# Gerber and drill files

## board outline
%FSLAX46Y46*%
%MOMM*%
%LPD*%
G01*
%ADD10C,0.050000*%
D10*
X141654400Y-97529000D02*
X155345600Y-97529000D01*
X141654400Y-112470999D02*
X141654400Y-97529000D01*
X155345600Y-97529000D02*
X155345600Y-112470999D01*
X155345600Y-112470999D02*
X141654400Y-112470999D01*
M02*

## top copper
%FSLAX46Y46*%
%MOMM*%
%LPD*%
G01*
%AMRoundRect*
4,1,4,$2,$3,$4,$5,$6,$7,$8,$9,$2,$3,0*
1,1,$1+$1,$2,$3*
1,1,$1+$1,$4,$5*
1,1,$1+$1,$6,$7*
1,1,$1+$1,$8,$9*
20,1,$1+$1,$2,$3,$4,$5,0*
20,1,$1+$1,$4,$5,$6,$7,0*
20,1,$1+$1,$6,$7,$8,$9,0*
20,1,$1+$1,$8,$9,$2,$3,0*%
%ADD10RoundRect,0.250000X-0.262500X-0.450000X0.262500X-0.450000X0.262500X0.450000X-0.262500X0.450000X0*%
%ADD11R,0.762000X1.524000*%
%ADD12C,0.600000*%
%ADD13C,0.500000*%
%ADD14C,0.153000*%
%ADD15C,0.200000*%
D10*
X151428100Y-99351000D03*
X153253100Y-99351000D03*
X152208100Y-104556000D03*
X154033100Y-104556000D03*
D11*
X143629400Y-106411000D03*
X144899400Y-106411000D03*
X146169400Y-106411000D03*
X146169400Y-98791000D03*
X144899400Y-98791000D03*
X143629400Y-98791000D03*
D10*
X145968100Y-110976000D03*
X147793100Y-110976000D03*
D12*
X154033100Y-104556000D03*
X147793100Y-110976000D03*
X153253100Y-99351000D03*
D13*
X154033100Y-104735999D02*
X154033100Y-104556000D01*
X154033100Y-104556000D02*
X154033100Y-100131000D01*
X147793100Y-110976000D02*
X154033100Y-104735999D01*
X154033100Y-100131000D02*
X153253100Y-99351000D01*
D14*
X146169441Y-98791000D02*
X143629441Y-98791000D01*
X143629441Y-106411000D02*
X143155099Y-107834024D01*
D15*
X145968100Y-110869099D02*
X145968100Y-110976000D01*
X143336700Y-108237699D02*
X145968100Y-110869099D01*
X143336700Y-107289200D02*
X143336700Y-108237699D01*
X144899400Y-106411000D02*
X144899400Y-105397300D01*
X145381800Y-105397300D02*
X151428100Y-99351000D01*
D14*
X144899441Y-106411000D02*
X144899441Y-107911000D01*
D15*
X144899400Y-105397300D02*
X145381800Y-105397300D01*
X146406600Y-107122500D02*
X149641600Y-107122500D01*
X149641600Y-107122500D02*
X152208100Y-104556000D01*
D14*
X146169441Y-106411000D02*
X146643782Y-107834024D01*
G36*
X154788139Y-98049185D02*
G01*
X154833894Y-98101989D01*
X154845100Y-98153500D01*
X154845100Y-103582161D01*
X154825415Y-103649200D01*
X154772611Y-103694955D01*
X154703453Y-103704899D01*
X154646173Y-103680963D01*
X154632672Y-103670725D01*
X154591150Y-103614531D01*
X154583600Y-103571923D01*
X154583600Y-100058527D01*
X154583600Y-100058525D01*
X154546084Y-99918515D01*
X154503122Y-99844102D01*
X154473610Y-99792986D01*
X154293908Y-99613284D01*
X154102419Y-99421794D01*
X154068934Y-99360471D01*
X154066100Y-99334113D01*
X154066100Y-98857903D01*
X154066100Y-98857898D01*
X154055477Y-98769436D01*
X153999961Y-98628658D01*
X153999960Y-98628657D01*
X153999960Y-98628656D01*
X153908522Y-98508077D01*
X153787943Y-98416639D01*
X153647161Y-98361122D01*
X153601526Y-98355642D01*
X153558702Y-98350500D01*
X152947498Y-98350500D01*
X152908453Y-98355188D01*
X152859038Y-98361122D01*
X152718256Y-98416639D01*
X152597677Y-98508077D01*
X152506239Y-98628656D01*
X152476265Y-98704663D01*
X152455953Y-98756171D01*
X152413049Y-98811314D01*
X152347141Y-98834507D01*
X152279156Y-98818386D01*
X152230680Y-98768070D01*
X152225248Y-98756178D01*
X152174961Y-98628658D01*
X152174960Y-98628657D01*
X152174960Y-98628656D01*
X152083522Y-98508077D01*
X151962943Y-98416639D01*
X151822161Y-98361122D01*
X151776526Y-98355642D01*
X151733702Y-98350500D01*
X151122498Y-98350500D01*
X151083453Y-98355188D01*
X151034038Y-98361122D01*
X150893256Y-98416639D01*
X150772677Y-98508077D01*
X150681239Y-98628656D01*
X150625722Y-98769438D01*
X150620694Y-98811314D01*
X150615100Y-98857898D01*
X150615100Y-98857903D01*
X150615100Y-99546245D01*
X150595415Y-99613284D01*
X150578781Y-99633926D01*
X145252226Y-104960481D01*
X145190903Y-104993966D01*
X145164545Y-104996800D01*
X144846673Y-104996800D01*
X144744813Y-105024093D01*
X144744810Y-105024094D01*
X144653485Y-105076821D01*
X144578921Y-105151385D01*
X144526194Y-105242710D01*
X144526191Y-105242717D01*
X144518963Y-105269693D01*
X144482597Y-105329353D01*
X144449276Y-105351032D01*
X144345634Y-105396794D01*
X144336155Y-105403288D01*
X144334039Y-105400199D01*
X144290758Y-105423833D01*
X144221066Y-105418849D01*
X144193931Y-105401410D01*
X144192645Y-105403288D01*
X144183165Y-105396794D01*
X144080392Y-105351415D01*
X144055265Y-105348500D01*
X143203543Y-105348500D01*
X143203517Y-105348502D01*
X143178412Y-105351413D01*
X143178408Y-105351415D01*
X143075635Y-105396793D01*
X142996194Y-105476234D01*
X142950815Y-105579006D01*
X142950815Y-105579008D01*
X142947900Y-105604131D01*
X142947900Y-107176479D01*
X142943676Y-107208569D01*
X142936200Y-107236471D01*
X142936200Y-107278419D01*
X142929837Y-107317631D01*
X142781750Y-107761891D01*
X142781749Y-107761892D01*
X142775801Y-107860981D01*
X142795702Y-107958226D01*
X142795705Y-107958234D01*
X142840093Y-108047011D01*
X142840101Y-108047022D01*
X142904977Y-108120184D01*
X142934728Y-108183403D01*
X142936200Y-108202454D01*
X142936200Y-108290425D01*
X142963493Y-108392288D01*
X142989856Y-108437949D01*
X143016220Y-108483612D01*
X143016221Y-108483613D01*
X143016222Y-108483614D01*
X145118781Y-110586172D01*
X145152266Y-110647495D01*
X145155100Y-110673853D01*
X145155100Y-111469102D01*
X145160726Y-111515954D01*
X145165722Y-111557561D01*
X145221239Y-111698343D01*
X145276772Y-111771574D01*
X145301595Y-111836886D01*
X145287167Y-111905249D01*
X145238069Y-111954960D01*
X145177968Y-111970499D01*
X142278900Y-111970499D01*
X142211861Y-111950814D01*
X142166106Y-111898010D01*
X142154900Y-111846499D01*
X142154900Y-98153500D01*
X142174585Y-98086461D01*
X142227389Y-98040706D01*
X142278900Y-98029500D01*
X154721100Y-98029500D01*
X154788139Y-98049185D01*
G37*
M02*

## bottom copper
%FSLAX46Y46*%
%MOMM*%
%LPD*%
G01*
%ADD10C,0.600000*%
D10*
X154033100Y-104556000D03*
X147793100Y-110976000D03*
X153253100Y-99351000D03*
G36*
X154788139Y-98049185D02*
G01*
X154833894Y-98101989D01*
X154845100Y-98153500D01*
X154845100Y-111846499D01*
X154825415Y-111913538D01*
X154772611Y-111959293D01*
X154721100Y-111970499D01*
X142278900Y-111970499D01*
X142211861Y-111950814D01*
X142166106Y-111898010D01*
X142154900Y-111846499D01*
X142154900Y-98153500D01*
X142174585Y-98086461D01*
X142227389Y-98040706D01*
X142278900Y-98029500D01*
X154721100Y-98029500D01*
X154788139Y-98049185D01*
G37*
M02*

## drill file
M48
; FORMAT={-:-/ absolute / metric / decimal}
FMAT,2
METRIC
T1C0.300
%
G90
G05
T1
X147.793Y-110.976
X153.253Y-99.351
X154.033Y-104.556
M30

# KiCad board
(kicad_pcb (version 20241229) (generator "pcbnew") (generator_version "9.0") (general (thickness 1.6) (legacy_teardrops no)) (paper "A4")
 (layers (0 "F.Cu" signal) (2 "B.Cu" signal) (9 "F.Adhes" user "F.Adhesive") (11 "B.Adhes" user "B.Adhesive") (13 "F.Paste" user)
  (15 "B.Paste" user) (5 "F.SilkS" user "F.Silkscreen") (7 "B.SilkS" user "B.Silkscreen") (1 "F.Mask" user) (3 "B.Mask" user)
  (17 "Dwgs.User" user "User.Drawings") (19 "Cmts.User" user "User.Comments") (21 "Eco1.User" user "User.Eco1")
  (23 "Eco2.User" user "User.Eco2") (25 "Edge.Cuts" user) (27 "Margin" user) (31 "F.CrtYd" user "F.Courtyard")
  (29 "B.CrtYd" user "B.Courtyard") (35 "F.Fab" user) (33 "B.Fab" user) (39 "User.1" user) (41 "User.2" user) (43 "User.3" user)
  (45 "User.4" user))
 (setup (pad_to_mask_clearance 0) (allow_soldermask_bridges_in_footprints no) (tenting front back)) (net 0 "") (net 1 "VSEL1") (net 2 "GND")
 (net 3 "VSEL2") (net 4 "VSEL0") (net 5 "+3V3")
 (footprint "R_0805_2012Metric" (layer "F.Cu") (at 152.3406 99.351)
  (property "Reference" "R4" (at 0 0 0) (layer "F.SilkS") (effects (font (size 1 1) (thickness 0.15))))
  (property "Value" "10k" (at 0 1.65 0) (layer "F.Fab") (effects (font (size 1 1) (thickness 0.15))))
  (pad "1" smd roundrect (at -0.9125 0) (size 1.025 1.4) (layers "F.Cu" "F.Mask" "F.Paste") (roundrect_rratio 0.243902) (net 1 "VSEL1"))
  (pad "2" smd roundrect (at 0.9125 0) (size 1.025 1.4) (layers "F.Cu" "F.Mask" "F.Paste") (roundrect_rratio 0.243902) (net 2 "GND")))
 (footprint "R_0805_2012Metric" (layer "F.Cu") (at 153.1206 104.556)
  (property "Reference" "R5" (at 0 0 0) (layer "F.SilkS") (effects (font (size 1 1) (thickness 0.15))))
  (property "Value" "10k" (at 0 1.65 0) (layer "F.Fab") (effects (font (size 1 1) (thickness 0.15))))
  (pad "1" smd roundrect (at -0.9125 0) (size 1.025 1.4) (layers "F.Cu" "F.Mask" "F.Paste") (roundrect_rratio 0.243902) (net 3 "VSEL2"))
  (pad "2" smd roundrect (at 0.9125 0) (size 1.025 1.4) (layers "F.Cu" "F.Mask" "F.Paste") (roundrect_rratio 0.243902) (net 2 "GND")))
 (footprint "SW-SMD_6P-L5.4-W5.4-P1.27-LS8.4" (layer "F.Cu") (at 144.8994 102.601)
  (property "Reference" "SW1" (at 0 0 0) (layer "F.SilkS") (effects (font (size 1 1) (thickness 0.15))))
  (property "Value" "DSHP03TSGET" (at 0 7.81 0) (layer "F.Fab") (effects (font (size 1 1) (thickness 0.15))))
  (pad "1" smd rect (at -1.27 3.81 90) (size 1.524 0.762) (layers "F.Cu" "F.Mask" "F.Paste") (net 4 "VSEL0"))
  (pad "2" smd rect (at 0 3.81 90) (size 1.524 0.762) (layers "F.Cu" "F.Mask" "F.Paste") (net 1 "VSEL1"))
  (pad "3" smd rect (at 1.27 3.81 90) (size 1.524 0.762) (layers "F.Cu" "F.Mask" "F.Paste") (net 3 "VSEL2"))
  (pad "4" smd rect (at 1.27 -3.81 90) (size 1.524 0.762) (layers "F.Cu" "F.Mask" "F.Paste") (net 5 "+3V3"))
  (pad "5" smd rect (at 0 -3.81 90) (size 1.524 0.762) (layers "F.Cu" "F.Mask" "F.Paste") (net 5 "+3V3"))
  (pad "6" smd rect (at -1.27 -3.81 90) (size 1.524 0.762) (layers "F.Cu" "F.Mask" "F.Paste") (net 5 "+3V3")))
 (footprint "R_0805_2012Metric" (layer "F.Cu") (at 146.8806 110.976)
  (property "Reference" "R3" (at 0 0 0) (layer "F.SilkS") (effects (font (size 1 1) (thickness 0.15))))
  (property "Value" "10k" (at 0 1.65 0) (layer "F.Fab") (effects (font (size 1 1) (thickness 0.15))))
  (pad "1" smd roundrect (at -0.9125 0) (size 1.025 1.4) (layers "F.Cu" "F.Mask" "F.Paste") (roundrect_rratio 0.243902) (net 4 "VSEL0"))
  (pad "2" smd roundrect (at 0.9125 0) (size 1.025 1.4) (layers "F.Cu" "F.Mask" "F.Paste") (roundrect_rratio 0.243902) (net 2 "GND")))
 (gr_line (start 141.6544 97.529) (end 155.3456 97.529) (stroke (width 0.05) (type default)) (layer "Edge.Cuts"))
 (gr_line (start 141.6544 112.470999) (end 141.6544 97.529) (stroke (width 0.05) (type default)) (layer "Edge.Cuts"))
 (gr_line (start 155.3456 97.529) (end 155.3456 112.470999) (stroke (width 0.05) (type default)) (layer "Edge.Cuts"))
 (gr_line (start 155.3456 112.470999) (end 141.6544 112.470999) (stroke (width 0.05) (type default)) (layer "Edge.Cuts"))
 (segment (start 154.0331 104.735999) (end 154.0331 104.556) (width 0.5) (layer "F.Cu") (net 2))
 (segment (start 154.0331 104.556) (end 154.0331 100.131) (width 0.5) (layer "F.Cu") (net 2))
 (segment (start 147.7931 110.976) (end 154.0331 104.735999) (width 0.5) (layer "F.Cu") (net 2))
 (segment (start 154.0331 100.131) (end 153.2531 99.351) (width 0.5) (layer "F.Cu") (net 2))
 (via (at 154.0331 104.556) (size 0.6) (drill 0.3) (layers "F.Cu" "B.Cu") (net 2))
 (via (at 147.7931 110.976) (size 0.6) (drill 0.3) (layers "F.Cu" "B.Cu") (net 2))
 (via (at 153.2531 99.351) (size 0.6) (drill 0.3) (layers "F.Cu" "B.Cu") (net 2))
 (segment (start 146.169441 98.791) (end 143.629441 98.791) (width 0.153) (layer "F.Cu") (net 5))
 (segment (start 143.629441 106.411) (end 143.155099 107.834024) (width 0.153) (layer "F.Cu") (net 4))
 (segment (start 145.9681 110.869099) (end 145.9681 110.976) (width 0.2) (layer "F.Cu") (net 4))
 (segment (start 143.3367 108.237699) (end 145.9681 110.869099) (width 0.2) (layer "F.Cu") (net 4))
 (segment (start 143.3367 107.2892) (end 143.3367 108.237699) (width 0.2) (layer "F.Cu") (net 4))
 (segment (start 144.8994 106.411) (end 144.8994 105.3973) (width 0.2) (layer "F.Cu") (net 1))
 (segment (start 145.3818 105.3973) (end 151.4281 99.351) (width 0.2) (layer "F.Cu") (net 1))
 (segment (start 144.899441 106.411) (end 144.899441 107.911) (width 0.153) (layer "F.Cu") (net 1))
 (segment (start 144.8994 105.3973) (end 145.3818 105.3973) (width 0.2) (layer "F.Cu") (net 1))
 (segment (start 146.4066 107.1225) (end 149.6416 107.1225) (width 0.2) (layer "F.Cu") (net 3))
 (segment (start 149.6416 107.1225) (end 152.2081 104.556) (width 0.2) (layer "F.Cu") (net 3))
 (segment (start 146.169441 106.411) (end 146.643782 107.834024) (width 0.153) (layer "F.Cu") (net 3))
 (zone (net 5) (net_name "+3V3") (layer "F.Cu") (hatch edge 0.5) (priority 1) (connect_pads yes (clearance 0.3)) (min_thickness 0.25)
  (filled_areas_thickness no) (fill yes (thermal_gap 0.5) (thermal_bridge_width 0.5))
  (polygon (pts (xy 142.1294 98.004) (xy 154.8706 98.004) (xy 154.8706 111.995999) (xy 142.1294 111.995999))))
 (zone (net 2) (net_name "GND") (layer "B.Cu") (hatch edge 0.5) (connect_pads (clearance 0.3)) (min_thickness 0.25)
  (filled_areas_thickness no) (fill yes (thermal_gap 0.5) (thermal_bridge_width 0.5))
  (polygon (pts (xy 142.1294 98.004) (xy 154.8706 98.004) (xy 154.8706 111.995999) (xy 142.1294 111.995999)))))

